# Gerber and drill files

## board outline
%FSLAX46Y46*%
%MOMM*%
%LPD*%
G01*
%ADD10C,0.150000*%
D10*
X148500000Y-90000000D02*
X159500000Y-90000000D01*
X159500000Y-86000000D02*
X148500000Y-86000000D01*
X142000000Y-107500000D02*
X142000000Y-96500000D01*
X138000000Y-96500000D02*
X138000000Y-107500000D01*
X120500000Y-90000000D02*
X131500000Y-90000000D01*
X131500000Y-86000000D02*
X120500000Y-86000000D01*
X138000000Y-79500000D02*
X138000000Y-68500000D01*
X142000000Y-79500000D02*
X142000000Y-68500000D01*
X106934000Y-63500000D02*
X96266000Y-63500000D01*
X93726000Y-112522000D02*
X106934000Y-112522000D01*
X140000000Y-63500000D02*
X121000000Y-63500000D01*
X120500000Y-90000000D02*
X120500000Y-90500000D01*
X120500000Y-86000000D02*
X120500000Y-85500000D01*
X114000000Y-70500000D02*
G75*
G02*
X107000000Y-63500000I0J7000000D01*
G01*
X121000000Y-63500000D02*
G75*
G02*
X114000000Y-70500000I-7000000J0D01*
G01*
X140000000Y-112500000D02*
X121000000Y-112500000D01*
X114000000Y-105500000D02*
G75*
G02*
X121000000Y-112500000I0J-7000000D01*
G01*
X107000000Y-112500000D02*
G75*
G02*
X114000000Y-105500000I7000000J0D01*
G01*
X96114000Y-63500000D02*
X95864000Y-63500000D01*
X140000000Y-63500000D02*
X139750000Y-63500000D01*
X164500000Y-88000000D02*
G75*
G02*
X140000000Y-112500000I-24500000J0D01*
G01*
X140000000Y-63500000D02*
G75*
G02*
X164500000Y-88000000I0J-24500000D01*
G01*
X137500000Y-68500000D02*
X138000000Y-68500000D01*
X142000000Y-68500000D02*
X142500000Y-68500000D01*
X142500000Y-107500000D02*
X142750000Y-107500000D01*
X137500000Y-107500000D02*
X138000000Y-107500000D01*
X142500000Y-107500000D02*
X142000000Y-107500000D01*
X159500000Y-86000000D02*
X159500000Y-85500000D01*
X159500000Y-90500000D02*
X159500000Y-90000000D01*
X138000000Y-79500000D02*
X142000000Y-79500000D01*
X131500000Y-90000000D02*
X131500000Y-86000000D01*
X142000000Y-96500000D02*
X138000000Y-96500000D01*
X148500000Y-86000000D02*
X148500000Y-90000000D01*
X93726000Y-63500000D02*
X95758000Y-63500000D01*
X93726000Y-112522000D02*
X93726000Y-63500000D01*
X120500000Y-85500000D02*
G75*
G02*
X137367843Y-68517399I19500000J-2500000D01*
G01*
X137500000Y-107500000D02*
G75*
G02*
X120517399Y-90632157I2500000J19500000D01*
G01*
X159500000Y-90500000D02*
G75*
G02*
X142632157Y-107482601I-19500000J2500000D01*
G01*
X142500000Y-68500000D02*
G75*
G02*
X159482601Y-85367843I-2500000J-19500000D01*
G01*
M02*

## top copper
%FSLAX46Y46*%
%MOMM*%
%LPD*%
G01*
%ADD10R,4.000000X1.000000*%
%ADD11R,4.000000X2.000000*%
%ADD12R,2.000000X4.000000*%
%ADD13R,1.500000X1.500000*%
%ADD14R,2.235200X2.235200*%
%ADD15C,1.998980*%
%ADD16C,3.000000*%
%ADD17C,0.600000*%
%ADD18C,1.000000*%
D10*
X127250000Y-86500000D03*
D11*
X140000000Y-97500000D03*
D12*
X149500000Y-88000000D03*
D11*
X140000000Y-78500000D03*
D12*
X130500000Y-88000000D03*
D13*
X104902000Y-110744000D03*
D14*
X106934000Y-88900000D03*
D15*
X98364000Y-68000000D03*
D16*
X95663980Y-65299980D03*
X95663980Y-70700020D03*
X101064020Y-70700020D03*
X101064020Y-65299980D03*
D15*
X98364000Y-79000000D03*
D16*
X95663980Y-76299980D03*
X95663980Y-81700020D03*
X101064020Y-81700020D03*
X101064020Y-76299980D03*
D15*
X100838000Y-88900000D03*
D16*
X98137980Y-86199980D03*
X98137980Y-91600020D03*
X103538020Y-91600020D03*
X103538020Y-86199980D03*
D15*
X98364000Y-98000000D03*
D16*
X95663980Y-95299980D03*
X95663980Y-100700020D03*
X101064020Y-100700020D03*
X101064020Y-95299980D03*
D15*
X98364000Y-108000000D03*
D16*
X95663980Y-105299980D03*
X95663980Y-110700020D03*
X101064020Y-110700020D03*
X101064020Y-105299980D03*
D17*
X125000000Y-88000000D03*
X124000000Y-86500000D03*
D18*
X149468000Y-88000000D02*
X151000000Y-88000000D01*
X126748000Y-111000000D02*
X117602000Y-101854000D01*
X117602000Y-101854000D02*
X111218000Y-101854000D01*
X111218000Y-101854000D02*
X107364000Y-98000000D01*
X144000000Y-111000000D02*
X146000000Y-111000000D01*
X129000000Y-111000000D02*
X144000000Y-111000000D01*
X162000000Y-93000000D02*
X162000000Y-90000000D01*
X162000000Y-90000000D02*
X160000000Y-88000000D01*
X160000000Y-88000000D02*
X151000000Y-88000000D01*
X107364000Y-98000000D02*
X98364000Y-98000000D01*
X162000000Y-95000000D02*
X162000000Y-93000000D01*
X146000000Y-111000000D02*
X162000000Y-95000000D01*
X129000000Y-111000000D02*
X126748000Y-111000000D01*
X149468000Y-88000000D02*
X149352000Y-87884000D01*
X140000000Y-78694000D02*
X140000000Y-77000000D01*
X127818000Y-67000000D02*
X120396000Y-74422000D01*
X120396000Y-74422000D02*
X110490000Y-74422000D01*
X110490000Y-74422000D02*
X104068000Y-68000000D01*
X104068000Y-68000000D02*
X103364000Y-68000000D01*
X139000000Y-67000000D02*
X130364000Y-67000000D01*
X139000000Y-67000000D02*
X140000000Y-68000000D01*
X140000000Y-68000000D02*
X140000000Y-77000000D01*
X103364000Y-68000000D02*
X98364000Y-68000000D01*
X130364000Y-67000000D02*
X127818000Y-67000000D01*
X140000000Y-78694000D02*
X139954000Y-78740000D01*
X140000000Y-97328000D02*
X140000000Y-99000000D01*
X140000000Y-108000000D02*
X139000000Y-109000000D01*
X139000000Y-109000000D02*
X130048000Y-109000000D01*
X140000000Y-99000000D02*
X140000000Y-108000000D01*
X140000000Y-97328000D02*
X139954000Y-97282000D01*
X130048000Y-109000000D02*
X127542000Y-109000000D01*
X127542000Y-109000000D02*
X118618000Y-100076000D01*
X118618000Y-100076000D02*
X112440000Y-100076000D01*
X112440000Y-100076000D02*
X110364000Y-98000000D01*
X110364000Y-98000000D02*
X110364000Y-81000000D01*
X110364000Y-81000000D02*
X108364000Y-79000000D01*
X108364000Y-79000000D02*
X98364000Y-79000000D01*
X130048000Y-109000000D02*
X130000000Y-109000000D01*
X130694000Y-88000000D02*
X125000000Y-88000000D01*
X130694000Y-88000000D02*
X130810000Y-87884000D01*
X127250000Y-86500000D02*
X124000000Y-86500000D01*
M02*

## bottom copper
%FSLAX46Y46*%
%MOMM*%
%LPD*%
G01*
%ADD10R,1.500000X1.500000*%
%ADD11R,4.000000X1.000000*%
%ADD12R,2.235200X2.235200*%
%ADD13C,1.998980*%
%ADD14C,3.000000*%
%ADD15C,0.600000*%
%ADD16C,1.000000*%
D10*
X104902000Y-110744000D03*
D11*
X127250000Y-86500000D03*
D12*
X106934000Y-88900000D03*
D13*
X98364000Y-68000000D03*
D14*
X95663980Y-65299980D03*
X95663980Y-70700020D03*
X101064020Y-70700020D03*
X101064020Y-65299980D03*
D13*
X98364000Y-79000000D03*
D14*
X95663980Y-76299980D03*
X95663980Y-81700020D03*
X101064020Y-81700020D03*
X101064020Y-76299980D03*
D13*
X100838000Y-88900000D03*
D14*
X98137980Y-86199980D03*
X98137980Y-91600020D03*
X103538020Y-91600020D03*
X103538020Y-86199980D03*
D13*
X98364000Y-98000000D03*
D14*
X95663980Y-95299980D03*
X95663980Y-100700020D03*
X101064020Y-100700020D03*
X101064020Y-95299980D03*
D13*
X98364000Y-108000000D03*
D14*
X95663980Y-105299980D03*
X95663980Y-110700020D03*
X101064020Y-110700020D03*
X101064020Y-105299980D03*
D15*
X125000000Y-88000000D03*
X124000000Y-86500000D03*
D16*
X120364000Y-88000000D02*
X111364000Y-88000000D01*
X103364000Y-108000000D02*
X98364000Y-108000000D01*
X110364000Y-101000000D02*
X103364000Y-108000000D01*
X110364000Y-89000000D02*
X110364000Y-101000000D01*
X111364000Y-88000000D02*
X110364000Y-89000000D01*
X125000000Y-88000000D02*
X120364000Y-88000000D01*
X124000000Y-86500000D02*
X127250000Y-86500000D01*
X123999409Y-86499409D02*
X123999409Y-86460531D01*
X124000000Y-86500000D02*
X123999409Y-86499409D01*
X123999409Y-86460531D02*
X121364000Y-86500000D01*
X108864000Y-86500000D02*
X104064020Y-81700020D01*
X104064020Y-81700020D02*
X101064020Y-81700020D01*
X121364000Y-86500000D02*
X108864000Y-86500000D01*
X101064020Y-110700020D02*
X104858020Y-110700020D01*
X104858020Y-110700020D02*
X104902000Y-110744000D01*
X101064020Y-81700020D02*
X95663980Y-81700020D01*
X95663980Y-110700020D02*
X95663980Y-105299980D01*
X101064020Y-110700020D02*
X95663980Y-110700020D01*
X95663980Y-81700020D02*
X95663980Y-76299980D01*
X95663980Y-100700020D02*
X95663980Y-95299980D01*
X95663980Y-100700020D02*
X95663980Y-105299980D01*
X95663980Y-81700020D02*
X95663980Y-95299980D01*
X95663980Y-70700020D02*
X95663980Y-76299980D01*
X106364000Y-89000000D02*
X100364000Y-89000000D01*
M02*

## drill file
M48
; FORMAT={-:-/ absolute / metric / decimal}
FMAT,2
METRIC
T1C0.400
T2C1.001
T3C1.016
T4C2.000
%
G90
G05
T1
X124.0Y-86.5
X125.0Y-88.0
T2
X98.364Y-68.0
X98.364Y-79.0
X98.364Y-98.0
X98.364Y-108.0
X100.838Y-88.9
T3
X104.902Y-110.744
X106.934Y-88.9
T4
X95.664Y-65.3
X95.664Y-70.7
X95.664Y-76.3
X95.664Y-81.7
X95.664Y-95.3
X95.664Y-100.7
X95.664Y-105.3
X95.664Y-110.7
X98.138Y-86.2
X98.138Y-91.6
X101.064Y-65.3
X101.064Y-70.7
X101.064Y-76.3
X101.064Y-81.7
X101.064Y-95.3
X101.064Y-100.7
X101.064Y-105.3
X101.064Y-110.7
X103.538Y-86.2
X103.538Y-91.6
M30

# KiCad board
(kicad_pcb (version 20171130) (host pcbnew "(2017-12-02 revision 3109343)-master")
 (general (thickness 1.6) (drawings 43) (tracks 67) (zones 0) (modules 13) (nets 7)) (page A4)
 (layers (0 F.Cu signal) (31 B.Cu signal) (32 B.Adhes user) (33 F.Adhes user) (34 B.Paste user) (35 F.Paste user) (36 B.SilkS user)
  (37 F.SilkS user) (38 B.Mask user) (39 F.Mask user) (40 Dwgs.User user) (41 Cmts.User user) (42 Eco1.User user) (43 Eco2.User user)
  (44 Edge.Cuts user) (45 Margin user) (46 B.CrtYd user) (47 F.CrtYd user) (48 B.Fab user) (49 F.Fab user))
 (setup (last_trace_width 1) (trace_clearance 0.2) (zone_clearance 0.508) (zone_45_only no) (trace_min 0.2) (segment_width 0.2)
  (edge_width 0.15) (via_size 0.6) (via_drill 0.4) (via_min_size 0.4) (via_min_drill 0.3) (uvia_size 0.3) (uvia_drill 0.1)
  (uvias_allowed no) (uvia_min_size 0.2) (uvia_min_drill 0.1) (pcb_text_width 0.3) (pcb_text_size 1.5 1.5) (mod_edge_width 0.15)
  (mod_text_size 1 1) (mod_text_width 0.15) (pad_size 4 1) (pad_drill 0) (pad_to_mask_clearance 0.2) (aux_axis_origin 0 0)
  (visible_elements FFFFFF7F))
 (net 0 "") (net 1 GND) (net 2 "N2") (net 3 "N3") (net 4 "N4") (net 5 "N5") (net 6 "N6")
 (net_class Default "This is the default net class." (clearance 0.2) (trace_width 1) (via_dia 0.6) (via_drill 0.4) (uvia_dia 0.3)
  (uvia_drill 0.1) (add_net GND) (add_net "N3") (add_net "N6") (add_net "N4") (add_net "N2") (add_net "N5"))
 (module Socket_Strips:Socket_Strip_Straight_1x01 (layer B.Cu) (at 127.25 86.5)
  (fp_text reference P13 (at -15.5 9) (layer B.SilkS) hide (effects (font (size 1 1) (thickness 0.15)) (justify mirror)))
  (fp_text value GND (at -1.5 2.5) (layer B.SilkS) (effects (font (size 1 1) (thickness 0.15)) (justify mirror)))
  (pad 1 smd rect (at 0 0) (size 4 1) (layers F.Cu B.Paste F.Mask) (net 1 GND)))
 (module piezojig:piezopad (layer F.Cu) (at 140 97.5 90)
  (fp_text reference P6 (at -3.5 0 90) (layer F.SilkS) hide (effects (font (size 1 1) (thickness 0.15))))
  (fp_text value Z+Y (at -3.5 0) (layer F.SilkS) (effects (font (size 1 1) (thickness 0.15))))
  (pad 1 smd rect (at 0 0 90) (size 2 4) (layers F.Cu F.Paste F.Mask) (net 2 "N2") (solder_mask_margin 0.0001) (solder_paste_margin -0.0001)
   (clearance 0.0001)))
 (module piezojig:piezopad (layer F.Cu) (at 149.5 88 180)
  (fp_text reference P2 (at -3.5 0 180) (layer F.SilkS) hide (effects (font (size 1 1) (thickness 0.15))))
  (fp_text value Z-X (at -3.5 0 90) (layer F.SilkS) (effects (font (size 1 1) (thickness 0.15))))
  (pad 1 smd rect (at 0 0 180) (size 2 4) (layers F.Cu F.Paste F.Mask) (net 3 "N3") (solder_mask_margin 0.0001)
   (solder_paste_margin -0.0001) (clearance 0.0001)))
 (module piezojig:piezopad (layer F.Cu) (at 140 78.5 90)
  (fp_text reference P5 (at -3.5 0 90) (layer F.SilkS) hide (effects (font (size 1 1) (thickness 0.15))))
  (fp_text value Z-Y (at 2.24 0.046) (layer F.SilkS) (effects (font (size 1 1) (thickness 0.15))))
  (pad 1 smd rect (at 0 0 90) (size 2 4) (layers F.Cu F.Paste F.Mask) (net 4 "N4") (solder_mask_margin 0.0001) (solder_paste_margin -0.0001)
   (clearance 0.0001)))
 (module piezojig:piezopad (layer F.Cu) (at 130.5 88)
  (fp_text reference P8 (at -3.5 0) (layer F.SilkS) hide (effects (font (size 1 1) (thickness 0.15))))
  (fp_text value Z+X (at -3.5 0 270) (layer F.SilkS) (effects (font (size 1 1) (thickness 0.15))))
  (pad 1 smd rect (at 0 0) (size 2 4) (layers F.Cu F.Paste F.Mask) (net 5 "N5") (solder_mask_margin 0.0001) (solder_paste_margin -0.0001)
   (clearance 0.0001)))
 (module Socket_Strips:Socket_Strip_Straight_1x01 (layer F.Cu) (at 104.902 110.744)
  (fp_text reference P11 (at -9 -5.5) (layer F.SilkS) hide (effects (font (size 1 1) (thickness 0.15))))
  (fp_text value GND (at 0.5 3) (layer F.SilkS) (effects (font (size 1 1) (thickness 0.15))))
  (pad 1 thru_hole rect (at 0 0) (size 1.5 1.5) (drill 1.016) (layers *.Cu *.Mask F.SilkS) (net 1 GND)))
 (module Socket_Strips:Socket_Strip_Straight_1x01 (layer F.Cu) (at 127.25 86.5)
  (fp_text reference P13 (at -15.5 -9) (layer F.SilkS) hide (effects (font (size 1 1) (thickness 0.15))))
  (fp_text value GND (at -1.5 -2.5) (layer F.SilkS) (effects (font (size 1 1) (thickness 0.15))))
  (pad 1 smd rect (at 0 0) (size 4 1) (layers B.Cu F.Paste B.Mask) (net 1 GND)))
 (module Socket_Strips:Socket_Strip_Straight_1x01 (layer F.Cu) (at 106.934 88.9)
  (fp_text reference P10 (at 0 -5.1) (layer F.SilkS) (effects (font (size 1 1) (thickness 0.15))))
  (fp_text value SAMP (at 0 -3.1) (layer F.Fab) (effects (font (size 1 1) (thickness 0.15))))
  (pad 1 thru_hole rect (at 0 0) (size 2.2352 2.2352) (drill 1.016) (layers *.Cu *.Mask) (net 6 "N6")))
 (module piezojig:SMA (layer F.Cu) (at 98.364 68 90)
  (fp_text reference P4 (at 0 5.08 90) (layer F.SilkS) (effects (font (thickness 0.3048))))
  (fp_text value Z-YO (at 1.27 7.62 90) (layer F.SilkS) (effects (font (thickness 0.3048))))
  (pad 1 thru_hole circle (at 0 0 90) (size 1.99898 1.99898) (drill 1.00076) (layers *.Cu *.Mask F.SilkS) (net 4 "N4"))
  (pad 3 thru_hole circle (at 2.70002 -2.70002 90) (size 3 3) (drill 2) (layers *.Cu *.Mask F.SilkS))
  (pad 2 thru_hole circle (at -2.70002 -2.70002 90) (size 3 3) (drill 2) (layers *.Cu *.Mask F.SilkS))
  (pad 5 thru_hole circle (at -2.70002 2.70002 90) (size 3 3) (drill 2) (layers *.Cu *.Mask F.SilkS))
  (pad 4 thru_hole circle (at 2.70002 2.70002 90) (size 3 3) (drill 2) (layers *.Cu *.Mask F.SilkS)))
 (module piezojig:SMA (layer F.Cu) (at 98.364 79 90)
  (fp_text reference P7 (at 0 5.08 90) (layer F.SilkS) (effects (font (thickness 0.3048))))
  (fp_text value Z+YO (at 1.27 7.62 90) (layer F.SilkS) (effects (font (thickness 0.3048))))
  (pad 1 thru_hole circle (at 0 0 90) (size 1.99898 1.99898) (drill 1.00076) (layers *.Cu *.Mask F.SilkS) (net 2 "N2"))
  (pad 3 thru_hole circle (at 2.70002 -2.70002 90) (size 3 3) (drill 2) (layers *.Cu *.Mask F.SilkS))
  (pad 2 thru_hole circle (at -2.70002 -2.70002 90) (size 3 3) (drill 2) (layers *.Cu *.Mask F.SilkS) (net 1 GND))
  (pad 5 thru_hole circle (at -2.70002 2.70002 90) (size 3 3) (drill 2) (layers *.Cu *.Mask F.SilkS))
  (pad 4 thru_hole circle (at 2.70002 2.70002 90) (size 3 3) (drill 2) (layers *.Cu *.Mask F.SilkS)))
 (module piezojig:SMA (layer F.Cu) (at 100.838 88.9 90)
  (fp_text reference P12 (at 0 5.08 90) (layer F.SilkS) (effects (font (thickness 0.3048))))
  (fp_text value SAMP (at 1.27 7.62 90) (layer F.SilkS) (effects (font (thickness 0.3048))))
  (pad 1 thru_hole circle (at 0 0 90) (size 1.99898 1.99898) (drill 1.00076) (layers *.Cu *.Mask F.SilkS) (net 6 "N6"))
  (pad 3 thru_hole circle (at 2.70002 -2.70002 90) (size 3 3) (drill 2) (layers *.Cu *.Mask F.SilkS))
  (pad 2 thru_hole circle (at -2.70002 -2.70002 90) (size 3 3) (drill 2) (layers *.Cu *.Mask F.SilkS))
  (pad 5 thru_hole circle (at -2.70002 2.70002 90) (size 3 3) (drill 2) (layers *.Cu *.Mask F.SilkS))
  (pad 4 thru_hole circle (at 2.70002 2.70002 90) (size 3 3) (drill 2) (layers *.Cu *.Mask F.SilkS)))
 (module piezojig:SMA (layer F.Cu) (at 98.364 98 90)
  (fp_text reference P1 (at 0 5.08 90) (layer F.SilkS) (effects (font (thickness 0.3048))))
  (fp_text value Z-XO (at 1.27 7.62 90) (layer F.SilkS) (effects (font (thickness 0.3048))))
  (pad 1 thru_hole circle (at 0 0 90) (size 1.99898 1.99898) (drill 1.00076) (layers *.Cu *.Mask F.SilkS) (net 3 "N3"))
  (pad 3 thru_hole circle (at 2.70002 -2.70002 90) (size 3 3) (drill 2) (layers *.Cu *.Mask F.SilkS))
  (pad 2 thru_hole circle (at -2.70002 -2.70002 90) (size 3 3) (drill 2) (layers *.Cu *.Mask F.SilkS) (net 1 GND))
  (pad 5 thru_hole circle (at -2.70002 2.70002 90) (size 3 3) (drill 2) (layers *.Cu *.Mask F.SilkS))
  (pad 4 thru_hole circle (at 2.70002 2.70002 90) (size 3 3) (drill 2) (layers *.Cu *.Mask F.SilkS)))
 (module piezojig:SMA (layer F.Cu) (at 98.364 108 90)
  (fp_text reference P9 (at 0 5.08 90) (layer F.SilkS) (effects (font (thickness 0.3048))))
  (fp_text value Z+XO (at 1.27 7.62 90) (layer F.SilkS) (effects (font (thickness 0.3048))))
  (pad 1 thru_hole circle (at 0 0 90) (size 1.99898 1.99898) (drill 1.00076) (layers *.Cu *.Mask F.SilkS) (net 5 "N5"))
  (pad 3 thru_hole circle (at 2.70002 -2.70002 90) (size 3 3) (drill 2) (layers *.Cu *.Mask F.SilkS))
  (pad 2 thru_hole circle (at -2.70002 -2.70002 90) (size 3 3) (drill 2) (layers *.Cu *.Mask F.SilkS) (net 1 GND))
  (pad 5 thru_hole circle (at -2.70002 2.70002 90) (size 3 3) (drill 2) (layers *.Cu *.Mask F.SilkS))
  (pad 4 thru_hole circle (at 2.70002 2.70002 90) (size 3 3) (drill 2) (layers *.Cu *.Mask F.SilkS)))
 (gr_line (start 148.5 90) (end 159.5 90) (angle 90) (layer Edge.Cuts) (width 0.15))
 (gr_line (start 159.5 86) (end 148.5 86) (angle 90) (layer Edge.Cuts) (width 0.15))
 (gr_line (start 142 107.5) (end 142 96.5) (angle 90) (layer Edge.Cuts) (width 0.15))
 (gr_line (start 138 96.5) (end 138 107.5) (angle 90) (layer Edge.Cuts) (width 0.15))
 (gr_line (start 120.5 90) (end 131.5 90) (angle 90) (layer Edge.Cuts) (width 0.15))
 (gr_line (start 131.5 86) (end 120.5 86) (angle 90) (layer Edge.Cuts) (width 0.15))
 (gr_line (start 138 79.5) (end 138 68.5) (angle 90) (layer Edge.Cuts) (width 0.15))
 (gr_line (start 142 79.5) (end 142 68.5) (angle 90) (layer Edge.Cuts) (width 0.15))
 (gr_line (start 106.934 63.5) (end 96.266 63.5) (angle 90) (layer Edge.Cuts) (width 0.15))
 (gr_line (start 93.726 112.522) (end 106.934 112.522) (angle 90) (layer Edge.Cuts) (width 0.15))
 (gr_line (start 140 63.5) (end 121 63.5) (angle 90) (layer Edge.Cuts) (width 0.15))
 (gr_line (start 120.5 90) (end 120.5 90.5) (angle 90) (layer Edge.Cuts) (width 0.15))
 (gr_line (start 120.5 86) (end 120.5 85.5) (angle 90) (layer Edge.Cuts) (width 0.15))
 (gr_arc (start 114 63.5) (end 114 70.5) (angle 90) (layer Edge.Cuts) (width 0.15))
 (gr_arc (start 114 63.5) (end 121 63.5) (angle 90) (layer Edge.Cuts) (width 0.15))
 (gr_line (start 140 112.5) (end 121 112.5) (angle 90) (layer Edge.Cuts) (width 0.15))
 (gr_arc (start 114 112.5) (end 114 105.5) (angle 90) (layer Edge.Cuts) (width 0.15))
 (gr_arc (start 114 112.5) (end 107 112.5) (angle 90) (layer Edge.Cuts) (width 0.15))
 (gr_line (start 96.114 63.5) (end 95.864 63.5) (angle 90) (layer Edge.Cuts) (width 0.15))
 (gr_line (start 140 63.5) (end 139.75 63.5) (angle 90) (layer Edge.Cuts) (width 0.15))
 (gr_arc (start 140 88) (end 164.5 88) (angle 90) (layer Edge.Cuts) (width 0.15))
 (gr_arc (start 140 88) (end 140 63.5) (angle 90) (layer Edge.Cuts) (width 0.15))
 (gr_line (start 137.5 68.5) (end 138 68.5) (angle 90) (layer Edge.Cuts) (width 0.15))
 (gr_line (start 142 68.5) (end 142.5 68.5) (angle 90) (layer Edge.Cuts) (width 0.15))
 (gr_line (start 142.5 107.5) (end 142.75 107.5) (angle 90) (layer Edge.Cuts) (width 0.15))
 (gr_line (start 137.5 107.5) (end 138 107.5) (angle 90) (layer Edge.Cuts) (width 0.15))
 (gr_line (start 142.5 107.5) (end 142 107.5) (angle 90) (layer Edge.Cuts) (width 0.15))
 (gr_line (start 159.5 86) (end 159.5 85.5) (angle 90) (layer Edge.Cuts) (width 0.15))
 (gr_line (start 159.5 90.5) (end 159.5 90) (angle 90) (layer Edge.Cuts) (width 0.15))
 (gr_line (start 138 79.5) (end 142 79.5) (angle 90) (layer Edge.Cuts) (width 0.15))
 (gr_line (start 131.5 90) (end 131.5 86) (angle 90) (layer Edge.Cuts) (width 0.15))
 (gr_line (start 142 96.5) (end 138 96.5) (angle 90) (layer Edge.Cuts) (width 0.15))
 (gr_line (start 148.5 86) (end 148.5 90) (angle 90) (layer Edge.Cuts) (width 0.15))
 (gr_line (start 93.726 63.5) (end 95.758 63.5) (angle 90) (layer Edge.Cuts) (width 0.15))
 (gr_line (start 93.726 112.522) (end 93.726 63.5) (angle 90) (layer Edge.Cuts) (width 0.15))
 (gr_arc (start 140 88) (end 120.5 85.5) (angle 75) (layer Edge.Cuts) (width 0.15))
 (gr_arc (start 140 88) (end 137.5 107.5) (angle 75) (layer Edge.Cuts) (width 0.15))
 (gr_arc (start 140 88) (end 159.5 90.5) (angle 75) (layer Edge.Cuts) (width 0.15))
 (gr_arc (start 140 88) (end 142.5 68.5) (angle 75) (layer Edge.Cuts) (width 0.15))
 (segment (start 149.468 88) (end 151 88) (width 1) (layer F.Cu) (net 3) (status 400000))
 (segment (start 126.748 111) (end 117.602 101.854) (width 1) (layer F.Cu) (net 3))
 (segment (start 117.602 101.854) (end 111.218 101.854) (width 1) (layer F.Cu) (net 3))
 (segment (start 111.218 101.854) (end 107.364 98) (width 1) (layer F.Cu) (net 3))
 (segment (start 144 111) (end 146 111) (width 1) (layer F.Cu) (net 3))
 (segment (start 129 111) (end 144 111) (width 1) (layer F.Cu) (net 3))
 (segment (start 162 93) (end 162 90) (width 1) (layer F.Cu) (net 3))
 (segment (start 162 90) (end 160 88) (width 1) (layer F.Cu) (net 3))
 (segment (start 160 88) (end 151 88) (width 1) (layer F.Cu) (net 3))
 (segment (start 107.364 98) (end 98.364 98) (width 1) (layer F.Cu) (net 3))
 (segment (start 162 95) (end 162 93) (width 1) (layer F.Cu) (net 3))
 (segment (start 146 111) (end 162 95) (width 1) (layer F.Cu) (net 3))
 (segment (start 129 111) (end 126.748 111) (width 1) (layer F.Cu) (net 3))
 (segment (start 149.468 88) (end 149.352 87.884) (width 1) (layer F.Cu) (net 3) (status C00000))
 (segment (start 140 78.694) (end 140 77) (width 1) (layer F.Cu) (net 4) (status 400000))
 (segment (start 127.818 67) (end 120.396 74.422) (width 1) (layer F.Cu) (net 4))
 (segment (start 120.396 74.422) (end 110.49 74.422) (width 1) (layer F.Cu) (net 4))
 (segment (start 110.49 74.422) (end 104.068 68) (width 1) (layer F.Cu) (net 4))
 (segment (start 104.068 68) (end 103.364 68) (width 1) (layer F.Cu) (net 4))
 (segment (start 139 67) (end 130.364 67) (width 1) (layer F.Cu) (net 4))
 (segment (start 139 67) (end 140 68) (width 1) (layer F.Cu) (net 4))
 (segment (start 140 68) (end 140 77) (width 1) (layer F.Cu) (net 4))
 (segment (start 103.364 68) (end 98.364 68) (width 1) (layer F.Cu) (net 4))
 (segment (start 130.364 67) (end 127.818 67) (width 1) (layer F.Cu) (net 4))
 (segment (start 140 78.694) (end 139.954 78.74) (width 1) (layer F.Cu) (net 4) (status C00000))
 (segment (start 140 97.328) (end 140 99) (width 1) (layer F.Cu) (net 2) (status 400000))
 (segment (start 140 108) (end 139 109) (width 1) (layer F.Cu) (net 2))
 (segment (start 139 109) (end 130.048 109) (width 1) (layer F.Cu) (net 2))
 (segment (start 140 99) (end 140 108) (width 1) (layer F.Cu) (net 2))
 (segment (start 140 97.328) (end 139.954 97.282) (width 1) (layer F.Cu) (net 2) (status C00000))
 (segment (start 130.048 109) (end 127.542 109) (width 1) (layer F.Cu) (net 2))
 (segment (start 127.542 109) (end 118.618 100.076) (width 1) (layer F.Cu) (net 2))
 (segment (start 118.618 100.076) (end 112.44 100.076) (width 1) (layer F.Cu) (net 2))
 (segment (start 112.44 100.076) (end 110.364 98) (width 1) (layer F.Cu) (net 2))
 (segment (start 110.364 98) (end 110.364 81) (width 1) (layer F.Cu) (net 2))
 (segment (start 110.364 81) (end 108.364 79) (width 1) (layer F.Cu) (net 2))
 (segment (start 108.364 79) (end 98.364 79) (width 1) (layer F.Cu) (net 2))
 (segment (start 130.048 109) (end 130 109) (width 1) (layer F.Cu) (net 2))
 (segment (start 130.694 88) (end 125 88) (width 1) (layer F.Cu) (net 5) (status 400000))
 (via (at 125 88) (size 0.6) (drill 0.4) (layers F.Cu B.Cu) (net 5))
 (segment (start 120.364 88) (end 111.364 88) (width 1) (layer B.Cu) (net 5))
 (segment (start 103.364 108) (end 98.364 108) (width 1) (layer B.Cu) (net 5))
 (segment (start 110.364 101) (end 103.364 108) (width 1) (layer B.Cu) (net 5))
 (segment (start 110.364 89) (end 110.364 101) (width 1) (layer B.Cu) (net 5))
 (segment (start 111.364 88) (end 110.364 89) (width 1) (layer B.Cu) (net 5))
 (segment (start 125 88) (end 120.364 88) (width 1) (layer B.Cu) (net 5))
 (segment (start 130.694 88) (end 130.81 87.884) (width 1) (layer F.Cu) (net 5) (status C00000))
 (segment (start 124 86.5) (end 127.25 86.5) (width 1) (layer B.Cu) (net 1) (status 800000))
 (segment (start 127.25 86.5) (end 124 86.5) (width 1) (layer F.Cu) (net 1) (status 400010))
 (segment (start 123.999409 86.499409) (end 123.999409 86.460531) (width 1) (layer B.Cu) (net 1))
 (segment (start 124 86.5) (end 123.999409 86.499409) (width 1) (layer B.Cu) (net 1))
 (via (at 124 86.5) (size 0.6) (drill 0.4) (layers F.Cu B.Cu) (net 1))
 (segment (start 123.999409 86.460531) (end 121.364 86.5) (width 1) (layer B.Cu) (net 1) (status 10))
 (segment (start 108.864 86.5) (end 104.06402 81.70002) (width 1) (layer B.Cu) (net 1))
 (segment (start 104.06402 81.70002) (end 101.06402 81.70002) (width 1) (layer B.Cu) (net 1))
 (segment (start 121.364 86.5) (end 108.864 86.5) (width 1) (layer B.Cu) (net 1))
 (segment (start 101.06402 110.70002) (end 104.85802 110.70002) (width 1) (layer B.Cu) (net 1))
 (segment (start 104.85802 110.70002) (end 104.902 110.744) (width 1) (layer B.Cu) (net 1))
 (segment (start 101.06402 81.70002) (end 95.66398 81.70002) (width 1) (layer B.Cu) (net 1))
 (segment (start 95.66398 110.70002) (end 95.66398 105.29998) (width 1) (layer B.Cu) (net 1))
 (segment (start 101.06402 110.70002) (end 95.66398 110.70002) (width 1) (layer B.Cu) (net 1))
 (segment (start 95.66398 81.70002) (end 95.66398 76.29998) (width 1) (layer B.Cu) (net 1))
 (segment (start 95.66398 100.70002) (end 95.66398 95.29998) (width 1) (layer B.Cu) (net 1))
 (segment (start 95.66398 100.70002) (end 95.66398 105.29998) (width 1) (layer B.Cu) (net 1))
 (segment (start 95.66398 81.70002) (end 95.66398 95.29998) (width 1) (layer B.Cu) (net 1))
 (segment (start 95.66398 70.70002) (end 95.66398 76.29998) (width 1) (layer B.Cu) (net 1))
 (segment (start 106.364 89) (end 100.364 89) (width 1) (layer B.Cu) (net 6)))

